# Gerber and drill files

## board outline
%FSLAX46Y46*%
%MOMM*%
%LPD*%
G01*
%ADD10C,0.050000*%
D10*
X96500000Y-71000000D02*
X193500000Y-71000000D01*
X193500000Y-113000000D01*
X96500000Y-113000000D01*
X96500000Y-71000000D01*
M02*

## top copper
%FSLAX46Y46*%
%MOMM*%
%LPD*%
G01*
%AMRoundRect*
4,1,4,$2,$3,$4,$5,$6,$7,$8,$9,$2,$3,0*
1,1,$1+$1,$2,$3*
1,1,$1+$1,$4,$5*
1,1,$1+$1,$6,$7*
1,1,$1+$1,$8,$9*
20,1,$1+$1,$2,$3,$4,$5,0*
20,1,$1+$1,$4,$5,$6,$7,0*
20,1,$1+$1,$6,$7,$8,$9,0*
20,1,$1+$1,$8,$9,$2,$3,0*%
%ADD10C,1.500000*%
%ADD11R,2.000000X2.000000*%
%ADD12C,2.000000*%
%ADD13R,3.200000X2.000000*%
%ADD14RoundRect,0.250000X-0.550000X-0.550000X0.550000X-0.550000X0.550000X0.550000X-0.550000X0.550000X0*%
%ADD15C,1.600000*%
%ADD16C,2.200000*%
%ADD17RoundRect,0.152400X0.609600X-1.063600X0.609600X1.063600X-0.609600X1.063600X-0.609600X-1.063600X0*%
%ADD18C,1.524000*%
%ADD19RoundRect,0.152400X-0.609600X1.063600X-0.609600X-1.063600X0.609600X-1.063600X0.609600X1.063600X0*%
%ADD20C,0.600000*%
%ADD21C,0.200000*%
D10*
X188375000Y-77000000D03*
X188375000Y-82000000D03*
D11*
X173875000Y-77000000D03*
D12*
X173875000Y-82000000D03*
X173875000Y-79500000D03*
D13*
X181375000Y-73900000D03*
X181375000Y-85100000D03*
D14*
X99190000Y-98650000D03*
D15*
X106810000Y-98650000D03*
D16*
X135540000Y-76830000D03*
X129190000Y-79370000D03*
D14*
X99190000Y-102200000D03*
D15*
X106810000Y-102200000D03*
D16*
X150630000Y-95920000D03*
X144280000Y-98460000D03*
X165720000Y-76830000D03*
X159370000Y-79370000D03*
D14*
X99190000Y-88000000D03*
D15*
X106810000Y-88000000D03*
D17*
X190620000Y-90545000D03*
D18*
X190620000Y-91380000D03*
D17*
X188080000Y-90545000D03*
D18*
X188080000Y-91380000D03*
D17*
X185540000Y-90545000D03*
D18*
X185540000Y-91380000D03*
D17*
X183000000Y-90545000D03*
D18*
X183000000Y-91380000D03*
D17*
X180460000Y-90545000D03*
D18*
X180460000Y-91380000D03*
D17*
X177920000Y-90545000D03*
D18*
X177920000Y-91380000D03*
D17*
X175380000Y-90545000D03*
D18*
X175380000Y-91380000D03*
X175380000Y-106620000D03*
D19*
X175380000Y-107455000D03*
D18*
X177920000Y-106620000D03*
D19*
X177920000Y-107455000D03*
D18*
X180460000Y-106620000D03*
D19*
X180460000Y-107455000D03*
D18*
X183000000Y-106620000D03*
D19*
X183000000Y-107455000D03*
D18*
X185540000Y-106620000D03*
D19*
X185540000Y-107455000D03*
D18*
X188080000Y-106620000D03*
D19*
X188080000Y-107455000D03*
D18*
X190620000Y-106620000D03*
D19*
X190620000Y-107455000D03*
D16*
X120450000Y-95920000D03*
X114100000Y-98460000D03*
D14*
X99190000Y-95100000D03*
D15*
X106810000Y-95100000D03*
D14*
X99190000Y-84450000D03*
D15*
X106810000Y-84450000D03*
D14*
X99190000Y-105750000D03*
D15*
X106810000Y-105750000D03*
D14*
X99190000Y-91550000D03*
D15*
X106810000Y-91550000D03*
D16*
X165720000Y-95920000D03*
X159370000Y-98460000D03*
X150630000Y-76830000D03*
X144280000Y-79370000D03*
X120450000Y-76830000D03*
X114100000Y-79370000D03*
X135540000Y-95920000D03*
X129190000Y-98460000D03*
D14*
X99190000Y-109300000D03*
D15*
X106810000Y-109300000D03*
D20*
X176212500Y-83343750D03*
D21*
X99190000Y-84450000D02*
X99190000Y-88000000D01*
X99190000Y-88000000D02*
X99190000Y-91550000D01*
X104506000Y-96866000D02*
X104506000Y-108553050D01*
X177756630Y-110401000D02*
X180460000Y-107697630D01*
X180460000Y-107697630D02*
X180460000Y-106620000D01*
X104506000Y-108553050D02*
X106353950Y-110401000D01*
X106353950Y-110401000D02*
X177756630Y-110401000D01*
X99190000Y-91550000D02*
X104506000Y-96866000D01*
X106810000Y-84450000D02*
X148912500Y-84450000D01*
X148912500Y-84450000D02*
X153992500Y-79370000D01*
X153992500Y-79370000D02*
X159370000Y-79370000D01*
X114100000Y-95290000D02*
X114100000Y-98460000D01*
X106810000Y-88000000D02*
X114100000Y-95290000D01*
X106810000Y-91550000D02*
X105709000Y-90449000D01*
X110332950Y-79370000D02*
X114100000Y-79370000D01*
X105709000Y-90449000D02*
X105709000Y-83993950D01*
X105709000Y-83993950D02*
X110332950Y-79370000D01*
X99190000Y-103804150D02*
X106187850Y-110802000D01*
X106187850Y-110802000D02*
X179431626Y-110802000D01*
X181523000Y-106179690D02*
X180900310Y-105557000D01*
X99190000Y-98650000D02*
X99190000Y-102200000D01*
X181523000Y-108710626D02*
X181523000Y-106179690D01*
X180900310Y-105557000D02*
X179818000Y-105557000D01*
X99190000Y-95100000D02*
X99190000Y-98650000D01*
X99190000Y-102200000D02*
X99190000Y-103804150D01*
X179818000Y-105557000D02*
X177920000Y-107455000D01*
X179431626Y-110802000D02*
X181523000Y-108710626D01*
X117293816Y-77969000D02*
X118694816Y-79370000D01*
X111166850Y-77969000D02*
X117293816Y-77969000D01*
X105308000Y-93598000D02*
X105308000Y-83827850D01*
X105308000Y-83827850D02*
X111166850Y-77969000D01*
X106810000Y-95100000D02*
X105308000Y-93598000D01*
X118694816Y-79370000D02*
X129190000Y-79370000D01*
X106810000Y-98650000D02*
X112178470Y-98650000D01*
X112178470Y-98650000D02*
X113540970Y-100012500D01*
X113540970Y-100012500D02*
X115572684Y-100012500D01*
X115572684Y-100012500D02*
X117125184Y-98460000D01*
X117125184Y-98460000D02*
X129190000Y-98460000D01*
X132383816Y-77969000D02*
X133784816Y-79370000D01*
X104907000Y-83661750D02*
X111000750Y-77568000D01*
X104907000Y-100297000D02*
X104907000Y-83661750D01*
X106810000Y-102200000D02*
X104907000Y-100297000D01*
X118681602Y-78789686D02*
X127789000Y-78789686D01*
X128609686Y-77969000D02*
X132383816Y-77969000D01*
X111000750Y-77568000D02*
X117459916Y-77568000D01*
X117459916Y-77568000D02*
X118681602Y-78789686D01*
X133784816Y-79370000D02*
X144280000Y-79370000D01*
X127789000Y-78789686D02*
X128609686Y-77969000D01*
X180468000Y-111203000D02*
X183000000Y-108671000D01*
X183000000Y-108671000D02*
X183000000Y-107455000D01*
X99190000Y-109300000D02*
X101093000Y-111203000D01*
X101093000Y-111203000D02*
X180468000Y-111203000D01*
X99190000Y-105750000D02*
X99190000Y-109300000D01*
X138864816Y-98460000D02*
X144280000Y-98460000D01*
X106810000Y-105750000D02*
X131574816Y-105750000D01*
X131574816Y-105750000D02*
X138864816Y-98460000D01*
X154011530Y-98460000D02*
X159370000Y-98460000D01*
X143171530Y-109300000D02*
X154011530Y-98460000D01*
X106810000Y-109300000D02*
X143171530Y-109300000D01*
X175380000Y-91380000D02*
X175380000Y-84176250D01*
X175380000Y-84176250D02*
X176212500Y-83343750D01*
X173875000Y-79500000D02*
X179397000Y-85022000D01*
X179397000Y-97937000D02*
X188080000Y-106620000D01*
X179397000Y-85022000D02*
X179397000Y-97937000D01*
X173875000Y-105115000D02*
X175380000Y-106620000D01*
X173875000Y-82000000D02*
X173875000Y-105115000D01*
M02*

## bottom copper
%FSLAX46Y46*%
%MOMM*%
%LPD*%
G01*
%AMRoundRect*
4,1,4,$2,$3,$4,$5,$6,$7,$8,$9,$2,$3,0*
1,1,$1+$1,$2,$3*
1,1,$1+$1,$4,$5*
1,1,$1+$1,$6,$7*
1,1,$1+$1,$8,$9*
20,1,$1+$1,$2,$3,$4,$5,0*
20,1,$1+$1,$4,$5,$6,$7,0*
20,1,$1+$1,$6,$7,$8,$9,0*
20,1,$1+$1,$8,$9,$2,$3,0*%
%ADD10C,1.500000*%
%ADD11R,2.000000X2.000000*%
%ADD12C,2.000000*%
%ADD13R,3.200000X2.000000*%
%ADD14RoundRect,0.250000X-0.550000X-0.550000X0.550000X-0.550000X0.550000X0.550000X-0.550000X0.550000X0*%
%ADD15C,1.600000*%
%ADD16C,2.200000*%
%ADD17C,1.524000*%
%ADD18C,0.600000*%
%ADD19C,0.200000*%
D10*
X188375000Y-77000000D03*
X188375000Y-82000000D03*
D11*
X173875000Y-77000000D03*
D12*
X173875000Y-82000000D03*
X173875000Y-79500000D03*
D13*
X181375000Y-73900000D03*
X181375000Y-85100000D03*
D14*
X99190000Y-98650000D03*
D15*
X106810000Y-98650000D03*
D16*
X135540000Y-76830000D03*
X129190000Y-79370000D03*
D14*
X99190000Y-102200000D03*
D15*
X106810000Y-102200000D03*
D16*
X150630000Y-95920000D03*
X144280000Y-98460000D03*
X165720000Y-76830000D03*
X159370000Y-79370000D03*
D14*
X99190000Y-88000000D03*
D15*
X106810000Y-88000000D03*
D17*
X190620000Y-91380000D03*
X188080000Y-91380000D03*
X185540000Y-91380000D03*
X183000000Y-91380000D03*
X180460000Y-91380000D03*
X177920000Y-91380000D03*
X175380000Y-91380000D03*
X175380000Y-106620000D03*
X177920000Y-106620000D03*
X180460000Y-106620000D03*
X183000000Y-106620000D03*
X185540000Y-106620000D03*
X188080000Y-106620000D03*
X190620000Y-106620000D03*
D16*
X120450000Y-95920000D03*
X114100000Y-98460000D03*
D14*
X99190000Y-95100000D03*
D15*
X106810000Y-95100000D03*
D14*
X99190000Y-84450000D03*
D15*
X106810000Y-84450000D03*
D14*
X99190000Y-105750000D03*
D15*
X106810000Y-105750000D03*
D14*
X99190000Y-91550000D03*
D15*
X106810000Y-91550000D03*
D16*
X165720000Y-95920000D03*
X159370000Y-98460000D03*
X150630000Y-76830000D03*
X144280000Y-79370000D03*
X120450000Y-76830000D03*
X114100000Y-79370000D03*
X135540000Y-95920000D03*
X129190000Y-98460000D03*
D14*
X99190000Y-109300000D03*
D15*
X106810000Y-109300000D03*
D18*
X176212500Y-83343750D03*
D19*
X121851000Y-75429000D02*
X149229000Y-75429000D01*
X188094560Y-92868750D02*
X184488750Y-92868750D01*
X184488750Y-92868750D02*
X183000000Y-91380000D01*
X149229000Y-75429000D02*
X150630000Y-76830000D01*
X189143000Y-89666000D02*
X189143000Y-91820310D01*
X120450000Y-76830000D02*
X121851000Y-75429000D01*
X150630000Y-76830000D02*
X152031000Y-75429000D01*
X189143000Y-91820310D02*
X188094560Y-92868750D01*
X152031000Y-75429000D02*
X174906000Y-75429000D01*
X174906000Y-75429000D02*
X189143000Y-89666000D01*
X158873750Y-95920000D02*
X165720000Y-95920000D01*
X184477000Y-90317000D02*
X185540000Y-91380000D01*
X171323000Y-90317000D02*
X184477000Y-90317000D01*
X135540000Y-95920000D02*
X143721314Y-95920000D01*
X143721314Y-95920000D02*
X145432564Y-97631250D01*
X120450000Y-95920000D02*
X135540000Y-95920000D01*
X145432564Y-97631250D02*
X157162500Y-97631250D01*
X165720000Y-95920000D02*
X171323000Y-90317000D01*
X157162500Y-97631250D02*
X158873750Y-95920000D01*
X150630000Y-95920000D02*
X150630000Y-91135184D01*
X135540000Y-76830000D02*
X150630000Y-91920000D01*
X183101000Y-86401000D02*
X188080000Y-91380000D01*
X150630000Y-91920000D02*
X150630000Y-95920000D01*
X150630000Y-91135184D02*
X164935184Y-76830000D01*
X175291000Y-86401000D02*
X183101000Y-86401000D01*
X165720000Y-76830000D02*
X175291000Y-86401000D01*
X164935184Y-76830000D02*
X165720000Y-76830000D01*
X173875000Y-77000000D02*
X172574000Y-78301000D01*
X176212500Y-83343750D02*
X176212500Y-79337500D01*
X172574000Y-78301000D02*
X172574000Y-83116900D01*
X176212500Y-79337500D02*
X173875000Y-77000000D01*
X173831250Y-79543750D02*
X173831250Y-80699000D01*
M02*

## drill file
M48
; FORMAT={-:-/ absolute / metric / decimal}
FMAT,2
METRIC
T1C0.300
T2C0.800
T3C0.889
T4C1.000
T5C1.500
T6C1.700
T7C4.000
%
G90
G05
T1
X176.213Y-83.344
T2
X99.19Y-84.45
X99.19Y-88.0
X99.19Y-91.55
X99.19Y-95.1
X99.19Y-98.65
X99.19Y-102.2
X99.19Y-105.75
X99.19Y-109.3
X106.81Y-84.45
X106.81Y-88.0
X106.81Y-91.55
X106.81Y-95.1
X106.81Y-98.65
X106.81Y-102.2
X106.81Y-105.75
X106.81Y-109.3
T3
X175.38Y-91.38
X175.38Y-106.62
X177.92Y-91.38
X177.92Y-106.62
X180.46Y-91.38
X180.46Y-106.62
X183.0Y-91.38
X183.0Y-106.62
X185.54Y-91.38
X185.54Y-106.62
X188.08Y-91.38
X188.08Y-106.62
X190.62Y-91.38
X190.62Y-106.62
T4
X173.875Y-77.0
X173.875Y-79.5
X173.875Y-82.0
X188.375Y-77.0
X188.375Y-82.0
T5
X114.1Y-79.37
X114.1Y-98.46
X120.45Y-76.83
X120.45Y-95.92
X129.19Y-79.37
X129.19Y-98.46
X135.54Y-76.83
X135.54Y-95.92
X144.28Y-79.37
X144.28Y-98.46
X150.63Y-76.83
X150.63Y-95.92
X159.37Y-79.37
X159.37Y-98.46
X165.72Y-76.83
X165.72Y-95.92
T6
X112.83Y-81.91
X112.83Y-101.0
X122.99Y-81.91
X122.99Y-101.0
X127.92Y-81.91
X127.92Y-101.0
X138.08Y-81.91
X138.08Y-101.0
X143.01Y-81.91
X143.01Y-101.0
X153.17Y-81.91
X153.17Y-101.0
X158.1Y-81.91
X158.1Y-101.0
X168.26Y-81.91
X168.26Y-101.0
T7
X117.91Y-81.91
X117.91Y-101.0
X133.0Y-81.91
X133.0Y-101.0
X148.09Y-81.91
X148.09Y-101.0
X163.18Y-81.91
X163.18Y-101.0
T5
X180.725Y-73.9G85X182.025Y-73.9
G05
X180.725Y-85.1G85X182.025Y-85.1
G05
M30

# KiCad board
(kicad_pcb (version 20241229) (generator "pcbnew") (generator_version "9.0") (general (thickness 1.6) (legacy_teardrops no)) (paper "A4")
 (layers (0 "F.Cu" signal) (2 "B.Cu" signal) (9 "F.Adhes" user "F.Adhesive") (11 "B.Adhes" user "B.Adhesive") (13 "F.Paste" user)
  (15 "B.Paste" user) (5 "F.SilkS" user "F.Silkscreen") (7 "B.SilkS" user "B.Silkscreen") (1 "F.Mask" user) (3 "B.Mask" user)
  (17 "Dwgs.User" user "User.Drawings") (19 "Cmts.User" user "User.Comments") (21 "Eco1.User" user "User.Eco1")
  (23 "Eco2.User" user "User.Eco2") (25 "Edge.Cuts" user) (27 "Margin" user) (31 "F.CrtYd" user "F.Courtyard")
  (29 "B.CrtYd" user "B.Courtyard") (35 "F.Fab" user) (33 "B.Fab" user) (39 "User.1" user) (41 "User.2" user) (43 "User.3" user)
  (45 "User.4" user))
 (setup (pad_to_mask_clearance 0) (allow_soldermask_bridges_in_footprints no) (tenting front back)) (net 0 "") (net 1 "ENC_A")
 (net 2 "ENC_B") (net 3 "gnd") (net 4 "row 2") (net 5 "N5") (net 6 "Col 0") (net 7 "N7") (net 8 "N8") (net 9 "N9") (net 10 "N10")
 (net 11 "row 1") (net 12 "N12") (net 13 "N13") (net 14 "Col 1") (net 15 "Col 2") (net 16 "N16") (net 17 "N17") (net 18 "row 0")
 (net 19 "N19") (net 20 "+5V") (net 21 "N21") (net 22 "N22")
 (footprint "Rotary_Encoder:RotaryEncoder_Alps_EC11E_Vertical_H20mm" (layer "F.Cu") (at 173.875 77)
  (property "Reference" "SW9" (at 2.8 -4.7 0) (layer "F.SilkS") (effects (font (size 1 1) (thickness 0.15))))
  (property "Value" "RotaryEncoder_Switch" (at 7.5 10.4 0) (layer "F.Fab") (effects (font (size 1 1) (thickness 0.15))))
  (pad "" thru_hole circle (at 14.5 0) (size 1.5 1.5) (drill 1) (layers "*.Cu" "*.Mask") (remove_unused_layers no))
  (pad "" thru_hole circle (at 14.5 5) (size 1.5 1.5) (drill 1) (layers "*.Cu" "*.Mask") (remove_unused_layers no))
  (pad "A" thru_hole rect (at 0 0) (size 2 2) (drill 1) (layers "*.Cu" "*.Mask") (remove_unused_layers no) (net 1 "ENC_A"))
  (pad "B" thru_hole circle (at 0 5) (size 2 2) (drill 1) (layers "*.Cu" "*.Mask") (remove_unused_layers no) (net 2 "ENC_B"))
  (pad "C" thru_hole circle (at 0 2.5) (size 2 2) (drill 1) (layers "*.Cu" "*.Mask") (remove_unused_layers no) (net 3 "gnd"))
  (pad "MP" thru_hole rect (at 7.5 -3.1) (size 3.2 2) (drill oval 2.8 1.5) (layers "*.Cu" "*.Mask") (remove_unused_layers no))
  (pad "MP" thru_hole rect (at 7.5 8.1) (size 3.2 2) (drill oval 2.8 1.5) (layers "*.Cu" "*.Mask") (remove_unused_layers no)))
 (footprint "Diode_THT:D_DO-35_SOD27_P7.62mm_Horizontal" (layer "F.Cu") (at 99.19 98.65)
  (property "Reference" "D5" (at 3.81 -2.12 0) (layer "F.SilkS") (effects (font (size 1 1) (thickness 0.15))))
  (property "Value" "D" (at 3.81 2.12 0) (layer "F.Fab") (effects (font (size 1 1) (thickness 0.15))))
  (pad "1" thru_hole roundrect (at 0 0) (size 1.6 1.6) (drill 0.8) (layers "*.Cu" "*.Mask") (remove_unused_layers no)
   (roundrect_rratio 0.15625) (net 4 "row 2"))
  (pad "2" thru_hole circle (at 7.62 0) (size 1.6 1.6) (drill 0.8) (layers "*.Cu" "*.Mask") (remove_unused_layers no) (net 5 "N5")))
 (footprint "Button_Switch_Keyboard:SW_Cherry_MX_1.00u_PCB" (layer "F.Cu") (at 135.54 76.83)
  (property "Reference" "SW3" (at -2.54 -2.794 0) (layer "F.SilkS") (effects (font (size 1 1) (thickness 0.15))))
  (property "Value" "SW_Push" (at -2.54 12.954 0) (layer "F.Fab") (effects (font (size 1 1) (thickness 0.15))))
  (pad "" np_thru_hole circle (at -7.62 5.08) (size 1.7 1.7) (drill 1.7) (layers "*.Cu" "*.Mask"))
  (pad "" np_thru_hole circle (at -2.54 5.08) (size 4 4) (drill 4) (layers "*.Cu" "*.Mask"))
  (pad "" np_thru_hole circle (at 2.54 5.08) (size 1.7 1.7) (drill 1.7) (layers "*.Cu" "*.Mask"))
  (pad "1" thru_hole circle (at 0 0) (size 2.2 2.2) (drill 1.5) (layers "*.Cu" "*.Mask") (remove_unused_layers no) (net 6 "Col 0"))
  (pad "2" thru_hole circle (at -6.35 2.54) (size 2.2 2.2) (drill 1.5) (layers "*.Cu" "*.Mask") (remove_unused_layers no) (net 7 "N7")))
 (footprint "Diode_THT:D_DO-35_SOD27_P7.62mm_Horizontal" (layer "F.Cu") (at 99.19 102.2)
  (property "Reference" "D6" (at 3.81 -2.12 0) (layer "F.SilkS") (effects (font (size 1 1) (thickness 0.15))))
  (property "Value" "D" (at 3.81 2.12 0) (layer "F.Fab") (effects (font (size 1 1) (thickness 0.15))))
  (pad "1" thru_hole roundrect (at 0 0) (size 1.6 1.6) (drill 0.8) (layers "*.Cu" "*.Mask") (remove_unused_layers no)
   (roundrect_rratio 0.15625) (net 4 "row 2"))
  (pad "2" thru_hole circle (at 7.62 0) (size 1.6 1.6) (drill 0.8) (layers "*.Cu" "*.Mask") (remove_unused_layers no) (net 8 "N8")))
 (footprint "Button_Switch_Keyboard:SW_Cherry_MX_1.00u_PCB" (layer "F.Cu") (at 150.63 95.92)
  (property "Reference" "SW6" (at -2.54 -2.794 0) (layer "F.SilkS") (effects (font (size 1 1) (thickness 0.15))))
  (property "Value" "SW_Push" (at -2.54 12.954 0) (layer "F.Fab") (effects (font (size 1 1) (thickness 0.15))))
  (pad "" np_thru_hole circle (at -7.62 5.08) (size 1.7 1.7) (drill 1.7) (layers "*.Cu" "*.Mask"))
  (pad "" np_thru_hole circle (at -2.54 5.08) (size 4 4) (drill 4) (layers "*.Cu" "*.Mask"))
  (pad "" np_thru_hole circle (at 2.54 5.08) (size 1.7 1.7) (drill 1.7) (layers "*.Cu" "*.Mask"))
  (pad "1" thru_hole circle (at 0 0) (size 2.2 2.2) (drill 1.5) (layers "*.Cu" "*.Mask") (remove_unused_layers no) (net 6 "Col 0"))
  (pad "2" thru_hole circle (at -6.35 2.54) (size 2.2 2.2) (drill 1.5) (layers "*.Cu" "*.Mask") (remove_unused_layers no) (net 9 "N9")))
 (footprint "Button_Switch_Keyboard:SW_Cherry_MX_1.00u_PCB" (layer "F.Cu") (at 165.72 76.83)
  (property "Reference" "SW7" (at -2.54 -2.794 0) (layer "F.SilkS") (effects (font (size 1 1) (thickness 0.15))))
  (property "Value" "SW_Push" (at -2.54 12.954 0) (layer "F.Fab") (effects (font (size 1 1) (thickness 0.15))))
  (pad "" np_thru_hole circle (at -7.62 5.08) (size 1.7 1.7) (drill 1.7) (layers "*.Cu" "*.Mask"))
  (pad "" np_thru_hole circle (at -2.54 5.08) (size 4 4) (drill 4) (layers "*.Cu" "*.Mask"))
  (pad "" np_thru_hole circle (at 2.54 5.08) (size 1.7 1.7) (drill 1.7) (layers "*.Cu" "*.Mask"))
  (pad "1" thru_hole circle (at 0 0) (size 2.2 2.2) (drill 1.5) (layers "*.Cu" "*.Mask") (remove_unused_layers no) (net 6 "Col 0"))
  (pad "2" thru_hole circle (at -6.35 2.54) (size 2.2 2.2) (drill 1.5) (layers "*.Cu" "*.Mask") (remove_unused_layers no) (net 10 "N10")))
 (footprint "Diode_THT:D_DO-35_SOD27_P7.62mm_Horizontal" (layer "F.Cu") (at 99.19 88)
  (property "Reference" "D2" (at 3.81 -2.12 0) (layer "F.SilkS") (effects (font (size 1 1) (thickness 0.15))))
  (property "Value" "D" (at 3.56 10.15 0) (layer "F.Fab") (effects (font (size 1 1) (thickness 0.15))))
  (pad "1" thru_hole roundrect (at 0 0) (size 1.6 1.6) (drill 0.8) (layers "*.Cu" "*.Mask") (remove_unused_layers no)
   (roundrect_rratio 0.15625) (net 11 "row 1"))
  (pad "2" thru_hole circle (at 7.62 0) (size 1.6 1.6) (drill 0.8) (layers "*.Cu" "*.Mask") (remove_unused_layers no) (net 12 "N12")))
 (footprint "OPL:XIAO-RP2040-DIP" (layer "F.Cu") (at 183 99 -90)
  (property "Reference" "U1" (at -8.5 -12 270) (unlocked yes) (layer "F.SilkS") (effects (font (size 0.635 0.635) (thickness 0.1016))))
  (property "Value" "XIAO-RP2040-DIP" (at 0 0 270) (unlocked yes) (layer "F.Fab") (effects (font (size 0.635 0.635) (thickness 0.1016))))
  (pad "1" smd roundrect (at -8.455 -7.62 90) (size 2.432 1.524) (layers "F.Cu" "F.Mask") (roundrect_rratio 0.1) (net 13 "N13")
   (thermal_bridge_angle 45))
  (pad "1" thru_hole circle (at -7.62 -7.62 90) (size 1.524 1.524) (drill 0.889) (layers "*.Cu" "*.Mask") (remove_unused_layers no)
   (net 13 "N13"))
  (pad "2" smd roundrect (at -8.455 -5.08 90) (size 2.432 1.524) (layers "F.Cu" "F.Mask") (roundrect_rratio 0.1) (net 6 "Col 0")
   (thermal_bridge_angle 45))
  (pad "2" thru_hole circle (at -7.62 -5.08 90) (size 1.524 1.524) (drill 0.889) (layers "*.Cu" "*.Mask") (remove_unused_layers no)
   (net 6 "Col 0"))
  (pad "3" smd roundrect (at -8.455 -2.54 90) (size 2.432 1.524) (layers "F.Cu" "F.Mask") (roundrect_rratio 0.1) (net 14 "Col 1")
   (thermal_bridge_angle 45))
  (pad "3" thru_hole circle (at -7.62 -2.54 90) (size 1.524 1.524) (drill 0.889) (layers "*.Cu" "*.Mask") (remove_unused_layers no)
   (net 14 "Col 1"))
  (pad "4" smd roundrect (at -8.455 0 90) (size 2.432 1.524) (layers "F.Cu" "F.Mask") (roundrect_rratio 0.1) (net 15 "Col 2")
   (thermal_bridge_angle 45))
  (pad "4" thru_hole circle (at -7.62 0 90) (size 1.524 1.524) (drill 0.889) (layers "*.Cu" "*.Mask") (remove_unused_layers no)
   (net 15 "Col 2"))
  (pad "5" smd roundrect (at -8.455 2.54 90) (size 2.432 1.524) (layers "F.Cu" "F.Mask") (roundrect_rratio 0.1) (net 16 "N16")
   (thermal_bridge_angle 45))
  (pad "5" thru_hole circle (at -7.62 2.54 90) (size 1.524 1.524) (drill 0.889) (layers "*.Cu" "*.Mask") (remove_unused_layers no)
   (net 16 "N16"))
  (pad "6" smd roundrect (at -8.455 5.08 90) (size 2.432 1.524) (layers "F.Cu" "F.Mask") (roundrect_rratio 0.1) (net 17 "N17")
   (thermal_bridge_angle 45))
  (pad "6" thru_hole circle (at -7.62 5.08 90) (size 1.524 1.524) (drill 0.889) (layers "*.Cu" "*.Mask") (remove_unused_layers no)
   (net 17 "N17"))
  (pad "7" smd roundrect (at -8.455 7.62 90) (size 2.432 1.524) (layers "F.Cu" "F.Mask") (roundrect_rratio 0.1) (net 1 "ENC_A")
   (thermal_bridge_angle 45))
  (pad "7" thru_hole circle (at -7.62 7.62 90) (size 1.524 1.524) (drill 0.889) (layers "*.Cu" "*.Mask") (remove_unused_layers no)
   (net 1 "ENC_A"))
  (pad "8" thru_hole circle (at 7.62 7.62 270) (size 1.524 1.524) (drill 0.889) (layers "*.Cu" "*.Mask") (remove_unused_layers no)
   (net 2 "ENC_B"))
  (pad "8" smd roundrect (at 8.455 7.62 270) (size 2.432 1.524) (layers "F.Cu" "F.Mask") (roundrect_rratio 0.1) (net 2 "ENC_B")
   (thermal_bridge_angle 45))
  (pad "9" thru_hole circle (at 7.62 5.08 270) (size 1.524 1.524) (drill 0.889) (layers "*.Cu" "*.Mask") (remove_unused_layers no)
   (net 4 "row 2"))
  (pad "9" smd roundrect (at 8.455 5.08 270) (size 2.432 1.524) (layers "F.Cu" "F.Mask") (roundrect_rratio 0.1) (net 4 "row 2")
   (thermal_bridge_angle 45))
  (pad "10" thru_hole circle (at 7.62 2.54 270) (size 1.524 1.524) (drill 0.889) (layers "*.Cu" "*.Mask") (remove_unused_layers no)
   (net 11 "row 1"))
  (pad "10" smd roundrect (at 8.455 2.54 270) (size 2.432 1.524) (layers "F.Cu" "F.Mask") (roundrect_rratio 0.1) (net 11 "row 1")
   (thermal_bridge_angle 45))
  (pad "11" thru_hole circle (at 7.62 0 270) (size 1.524 1.524) (drill 0.889) (layers "*.Cu" "*.Mask") (remove_unused_layers no)
   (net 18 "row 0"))
  (pad "11" smd roundrect (at 8.455 0 270) (size 2.432 1.524) (layers "F.Cu" "F.Mask") (roundrect_rratio 0.1) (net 18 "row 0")
   (thermal_bridge_angle 45))
  (pad "12" thru_hole circle (at 7.62 -2.54 270) (size 1.524 1.524) (drill 0.889) (layers "*.Cu" "*.Mask") (remove_unused_layers no)
   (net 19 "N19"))
  (pad "12" smd roundrect (at 8.455 -2.54 270) (size 2.432 1.524) (layers "F.Cu" "F.Mask") (roundrect_rratio 0.1) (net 19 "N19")
   (thermal_bridge_angle 45))
  (pad "13" thru_hole circle (at 7.62 -5.08 270) (size 1.524 1.524) (drill 0.889) (layers "*.Cu" "*.Mask") (remove_unused_layers no)
   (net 3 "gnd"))
  (pad "13" smd roundrect (at 8.455 -5.08 270) (size 2.432 1.524) (layers "F.Cu" "F.Mask") (roundrect_rratio 0.1) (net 3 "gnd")
   (thermal_bridge_angle 45))
  (pad "14" thru_hole circle (at 7.62 -7.62 270) (size 1.524 1.524) (drill 0.889) (layers "*.Cu" "*.Mask") (remove_unused_layers no)
   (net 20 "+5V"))
  (pad "14" smd roundrect (at 8.455 -7.62 270) (size 2.432 1.524) (layers "F.Cu" "F.Mask") (roundrect_rratio 0.1) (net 20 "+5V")
   (thermal_bridge_angle 45)))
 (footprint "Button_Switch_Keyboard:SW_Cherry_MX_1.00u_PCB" (layer "F.Cu") (at 120.45 95.92)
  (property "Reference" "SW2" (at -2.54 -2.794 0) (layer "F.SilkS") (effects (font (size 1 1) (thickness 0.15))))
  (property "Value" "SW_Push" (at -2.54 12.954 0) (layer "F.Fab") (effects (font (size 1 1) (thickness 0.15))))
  (pad "" np_thru_hole circle (at -7.62 5.08) (size 1.7 1.7) (drill 1.7) (layers "*.Cu" "*.Mask"))
  (pad "" np_thru_hole circle (at -2.54 5.08) (size 4 4) (drill 4) (layers "*.Cu" "*.Mask"))
  (pad "" np_thru_hole circle (at 2.54 5.08) (size 1.7 1.7) (drill 1.7) (layers "*.Cu" "*.Mask"))
  (pad "1" thru_hole circle (at 0 0) (size 2.2 2.2) (drill 1.5) (layers "*.Cu" "*.Mask") (remove_unused_layers no) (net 14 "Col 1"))
  (pad "2" thru_hole circle (at -6.35 2.54) (size 2.2 2.2) (drill 1.5) (layers "*.Cu" "*.Mask") (remove_unused_layers no) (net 12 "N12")))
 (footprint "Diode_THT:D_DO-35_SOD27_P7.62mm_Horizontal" (layer "F.Cu") (at 99.19 95.1)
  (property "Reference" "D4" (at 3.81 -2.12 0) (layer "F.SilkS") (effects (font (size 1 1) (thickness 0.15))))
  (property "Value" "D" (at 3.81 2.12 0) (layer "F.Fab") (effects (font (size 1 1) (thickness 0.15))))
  (pad "1" thru_hole roundrect (at 0 0) (size 1.6 1.6) (drill 0.8) (layers "*.Cu" "*.Mask") (remove_unused_layers no)
   (roundrect_rratio 0.15625) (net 4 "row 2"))
  (pad "2" thru_hole circle (at 7.62 0) (size 1.6 1.6) (drill 0.8) (layers "*.Cu" "*.Mask") (remove_unused_layers no) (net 7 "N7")))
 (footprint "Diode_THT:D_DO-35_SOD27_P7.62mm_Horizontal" (layer "F.Cu") (at 99.19 84.45)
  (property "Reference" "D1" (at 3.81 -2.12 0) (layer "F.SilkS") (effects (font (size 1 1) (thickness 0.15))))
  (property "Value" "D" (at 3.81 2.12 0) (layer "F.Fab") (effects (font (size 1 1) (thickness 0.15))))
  (pad "1" thru_hole roundrect (at 0 0) (size 1.6 1.6) (drill 0.8) (layers "*.Cu" "*.Mask") (remove_unused_layers no)
   (roundrect_rratio 0.15625) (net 11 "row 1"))
  (pad "2" thru_hole circle (at 7.62 0) (size 1.6 1.6) (drill 0.8) (layers "*.Cu" "*.Mask") (remove_unused_layers no) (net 10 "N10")))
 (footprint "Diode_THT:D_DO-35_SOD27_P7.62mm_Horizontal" (layer "F.Cu") (at 99.19 105.75)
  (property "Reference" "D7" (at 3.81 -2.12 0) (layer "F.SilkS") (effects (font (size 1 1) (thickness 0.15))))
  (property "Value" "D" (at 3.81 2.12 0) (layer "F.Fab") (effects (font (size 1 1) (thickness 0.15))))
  (pad "1" thru_hole roundrect (at 0 0) (size 1.6 1.6) (drill 0.8) (layers "*.Cu" "*.Mask") (remove_unused_layers no)
   (roundrect_rratio 0.15625) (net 18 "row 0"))
  (pad "2" thru_hole circle (at 7.62 0) (size 1.6 1.6) (drill 0.8) (layers "*.Cu" "*.Mask") (remove_unused_layers no) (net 9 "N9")))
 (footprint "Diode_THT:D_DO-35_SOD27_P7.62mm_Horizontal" (layer "F.Cu") (at 99.19 91.55)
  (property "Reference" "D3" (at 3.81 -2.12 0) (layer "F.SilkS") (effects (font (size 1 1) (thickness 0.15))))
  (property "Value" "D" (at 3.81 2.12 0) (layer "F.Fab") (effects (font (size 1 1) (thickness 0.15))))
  (pad "1" thru_hole roundrect (at 0 0) (size 1.6 1.6) (drill 0.8) (layers "*.Cu" "*.Mask") (remove_unused_layers no)
   (roundrect_rratio 0.15625) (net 11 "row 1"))
  (pad "2" thru_hole circle (at 7.62 0) (size 1.6 1.6) (drill 0.8) (layers "*.Cu" "*.Mask") (remove_unused_layers no) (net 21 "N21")))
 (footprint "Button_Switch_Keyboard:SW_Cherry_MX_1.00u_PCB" (layer "F.Cu") (at 165.72 95.92)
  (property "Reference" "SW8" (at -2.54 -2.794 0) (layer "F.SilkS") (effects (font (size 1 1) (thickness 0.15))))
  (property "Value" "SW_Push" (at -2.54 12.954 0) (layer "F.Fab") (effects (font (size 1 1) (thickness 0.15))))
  (pad "" np_thru_hole circle (at -7.62 5.08) (size 1.7 1.7) (drill 1.7) (layers "*.Cu" "*.Mask"))
  (pad "" np_thru_hole circle (at -2.54 5.08) (size 4 4) (drill 4) (layers "*.Cu" "*.Mask"))
  (pad "" np_thru_hole circle (at 2.54 5.08) (size 1.7 1.7) (drill 1.7) (layers "*.Cu" "*.Mask"))
  (pad "1" thru_hole circle (at 0 0) (size 2.2 2.2) (drill 1.5) (layers "*.Cu" "*.Mask") (remove_unused_layers no) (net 14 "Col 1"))
  (pad "2" thru_hole circle (at -6.35 2.54) (size 2.2 2.2) (drill 1.5) (layers "*.Cu" "*.Mask") (remove_unused_layers no) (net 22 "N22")))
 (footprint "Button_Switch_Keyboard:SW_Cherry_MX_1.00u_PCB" (layer "F.Cu") (at 150.63 76.83)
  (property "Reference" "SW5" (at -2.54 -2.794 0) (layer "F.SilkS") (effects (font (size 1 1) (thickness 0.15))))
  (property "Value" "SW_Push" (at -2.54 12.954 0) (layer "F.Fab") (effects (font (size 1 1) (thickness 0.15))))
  (pad "" np_thru_hole circle (at -7.62 5.08) (size 1.7 1.7) (drill 1.7) (layers "*.Cu" "*.Mask"))
  (pad "" np_thru_hole circle (at -2.54 5.08) (size 4 4) (drill 4) (layers "*.Cu" "*.Mask"))
  (pad "" np_thru_hole circle (at 2.54 5.08) (size 1.7 1.7) (drill 1.7) (layers "*.Cu" "*.Mask"))
  (pad "1" thru_hole circle (at 0 0) (size 2.2 2.2) (drill 1.5) (layers "*.Cu" "*.Mask") (remove_unused_layers no) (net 15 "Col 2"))
  (pad "2" thru_hole circle (at -6.35 2.54) (size 2.2 2.2) (drill 1.5) (layers "*.Cu" "*.Mask") (remove_unused_layers no) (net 8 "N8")))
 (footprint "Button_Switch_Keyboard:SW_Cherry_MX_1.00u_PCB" (layer "F.Cu") (at 120.45 76.83)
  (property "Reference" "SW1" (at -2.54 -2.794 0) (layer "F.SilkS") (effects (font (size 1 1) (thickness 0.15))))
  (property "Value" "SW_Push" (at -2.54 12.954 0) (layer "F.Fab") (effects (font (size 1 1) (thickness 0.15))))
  (pad "" np_thru_hole circle (at -7.62 5.08) (size 1.7 1.7) (drill 1.7) (layers "*.Cu" "*.Mask"))
  (pad "" np_thru_hole circle (at -2.54 5.08) (size 4 4) (drill 4) (layers "*.Cu" "*.Mask"))
  (pad "" np_thru_hole circle (at 2.54 5.08) (size 1.7 1.7) (drill 1.7) (layers "*.Cu" "*.Mask"))
  (pad "1" thru_hole circle (at 0 0) (size 2.2 2.2) (drill 1.5) (layers "*.Cu" "*.Mask") (remove_unused_layers no) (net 15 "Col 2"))
  (pad "2" thru_hole circle (at -6.35 2.54) (size 2.2 2.2) (drill 1.5) (layers "*.Cu" "*.Mask") (remove_unused_layers no) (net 21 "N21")))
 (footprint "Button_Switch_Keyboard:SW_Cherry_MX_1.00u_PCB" (layer "F.Cu") (at 135.54 95.92)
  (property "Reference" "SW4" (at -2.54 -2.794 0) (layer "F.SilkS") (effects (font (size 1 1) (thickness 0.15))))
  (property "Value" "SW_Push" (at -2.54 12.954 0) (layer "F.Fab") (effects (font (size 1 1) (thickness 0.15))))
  (pad "" np_thru_hole circle (at -7.62 5.08) (size 1.7 1.7) (drill 1.7) (layers "*.Cu" "*.Mask"))
  (pad "" np_thru_hole circle (at -2.54 5.08) (size 4 4) (drill 4) (layers "*.Cu" "*.Mask"))
  (pad "" np_thru_hole circle (at 2.54 5.08) (size 1.7 1.7) (drill 1.7) (layers "*.Cu" "*.Mask"))
  (pad "1" thru_hole circle (at 0 0) (size 2.2 2.2) (drill 1.5) (layers "*.Cu" "*.Mask") (remove_unused_layers no) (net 14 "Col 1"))
  (pad "2" thru_hole circle (at -6.35 2.54) (size 2.2 2.2) (drill 1.5) (layers "*.Cu" "*.Mask") (remove_unused_layers no) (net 5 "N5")))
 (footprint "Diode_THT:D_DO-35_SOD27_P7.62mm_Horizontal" (layer "F.Cu") (at 99.19 109.3)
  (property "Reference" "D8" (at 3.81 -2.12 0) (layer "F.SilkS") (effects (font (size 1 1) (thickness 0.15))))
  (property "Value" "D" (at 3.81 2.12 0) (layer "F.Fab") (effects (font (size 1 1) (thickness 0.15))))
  (pad "1" thru_hole roundrect (at 0 0) (size 1.6 1.6) (drill 0.8) (layers "*.Cu" "*.Mask") (remove_unused_layers no)
   (roundrect_rratio 0.15625) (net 18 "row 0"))
  (pad "2" thru_hole circle (at 7.62 0) (size 1.6 1.6) (drill 0.8) (layers "*.Cu" "*.Mask") (remove_unused_layers no) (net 22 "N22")))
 (gr_rect (start 96.5 71) (end 193.5 113) (stroke (width 0.05) (type default)) (fill no) (layer "Edge.Cuts"))
 (segment (start 99.19 84.45) (end 99.19 88) (width 0.2) (layer "F.Cu") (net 11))
 (segment (start 99.19 88) (end 99.19 91.55) (width 0.2) (layer "F.Cu") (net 11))
 (segment (start 104.506 96.866) (end 104.506 108.55305) (width 0.2) (layer "F.Cu") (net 11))
 (segment (start 177.75663 110.401) (end 180.46 107.69763) (width 0.2) (layer "F.Cu") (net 11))
 (segment (start 180.46 107.69763) (end 180.46 106.62) (width 0.2) (layer "F.Cu") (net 11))
 (segment (start 104.506 108.55305) (end 106.35395 110.401) (width 0.2) (layer "F.Cu") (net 11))
 (segment (start 106.35395 110.401) (end 177.75663 110.401) (width 0.2) (layer "F.Cu") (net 11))
 (segment (start 99.19 91.55) (end 104.506 96.866) (width 0.2) (layer "F.Cu") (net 11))
 (segment (start 106.81 84.45) (end 148.9125 84.45) (width 0.2) (layer "F.Cu") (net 10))
 (segment (start 148.9125 84.45) (end 153.9925 79.37) (width 0.2) (layer "F.Cu") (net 10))
 (segment (start 153.9925 79.37) (end 159.37 79.37) (width 0.2) (layer "F.Cu") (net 10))
 (segment (start 114.1 95.29) (end 114.1 98.46) (width 0.2) (layer "F.Cu") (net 12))
 (segment (start 106.81 88) (end 114.1 95.29) (width 0.2) (layer "F.Cu") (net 12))
 (segment (start 106.81 91.55) (end 105.709 90.449) (width 0.2) (layer "F.Cu") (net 21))
 (segment (start 110.33295 79.37) (end 114.1 79.37) (width 0.2) (layer "F.Cu") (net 21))
 (segment (start 105.709 90.449) (end 105.709 83.99395) (width 0.2) (layer "F.Cu") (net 21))
 (segment (start 105.709 83.99395) (end 110.33295 79.37) (width 0.2) (layer "F.Cu") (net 21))
 (segment (start 99.19 103.80415) (end 106.18785 110.802) (width 0.2) (layer "F.Cu") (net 4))
 (segment (start 106.18785 110.802) (end 179.431626 110.802) (width 0.2) (layer "F.Cu") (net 4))
 (segment (start 181.523 106.17969) (end 180.90031 105.557) (width 0.2) (layer "F.Cu") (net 4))
 (segment (start 99.19 98.65) (end 99.19 102.2) (width 0.2) (layer "F.Cu") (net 4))
 (segment (start 181.523 108.710626) (end 181.523 106.17969) (width 0.2) (layer "F.Cu") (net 4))
 (segment (start 180.90031 105.557) (end 179.818 105.557) (width 0.2) (layer "F.Cu") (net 4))
 (segment (start 99.19 95.1) (end 99.19 98.65) (width 0.2) (layer "F.Cu") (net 4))
 (segment (start 99.19 102.2) (end 99.19 103.80415) (width 0.2) (layer "F.Cu") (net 4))
 (segment (start 179.818 105.557) (end 177.92 107.455) (width 0.2) (layer "F.Cu") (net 4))
 (segment (start 179.431626 110.802) (end 181.523 108.710626) (width 0.2) (layer "F.Cu") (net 4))
 (segment (start 117.293816 77.969) (end 118.694816 79.37) (width 0.2) (layer "F.Cu") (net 7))
 (segment (start 111.16685 77.969) (end 117.293816 77.969) (width 0.2) (layer "F.Cu") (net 7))
 (segment (start 105.308 93.598) (end 105.308 83.82785) (width 0.2) (layer "F.Cu") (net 7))
 (segment (start 105.308 83.82785) (end 111.16685 77.969) (width 0.2) (layer "F.Cu") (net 7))
 (segment (start 106.81 95.1) (end 105.308 93.598) (width 0.2) (layer "F.Cu") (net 7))
 (segment (start 118.694816 79.37) (end 129.19 79.37) (width 0.2) (layer "F.Cu") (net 7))
 (segment (start 106.81 98.65) (end 112.17847 98.65) (width 0.2) (layer "F.Cu") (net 5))
 (segment (start 112.17847 98.65) (end 113.54097 100.0125) (width 0.2) (layer "F.Cu") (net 5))
 (segment (start 113.54097 100.0125) (end 115.572684 100.0125) (width 0.2) (layer "F.Cu") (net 5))
 (segment (start 115.572684 100.0125) (end 117.125184 98.46) (width 0.2) (layer "F.Cu") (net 5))
 (segment (start 117.125184 98.46) (end 129.19 98.46) (width 0.2) (layer "F.Cu") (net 5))
 (segment (start 132.383816 77.969) (end 133.784816 79.37) (width 0.2) (layer "F.Cu") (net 8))
 (segment (start 104.907 83.66175) (end 111.00075 77.568) (width 0.2) (layer "F.Cu") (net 8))
 (segment (start 104.907 100.297) (end 104.907 83.66175) (width 0.2) (layer "F.Cu") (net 8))
 (segment (start 106.81 102.2) (end 104.907 100.297) (width 0.2) (layer "F.Cu") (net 8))
 (segment (start 118.681602 78.789686) (end 127.789 78.789686) (width 0.2) (layer "F.Cu") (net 8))
 (segment (start 128.609686 77.969) (end 132.383816 77.969) (width 0.2) (layer "F.Cu") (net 8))
 (segment (start 111.00075 77.568) (end 117.459916 77.568) (width 0.2) (layer "F.Cu") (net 8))
 (segment (start 117.459916 77.568) (end 118.681602 78.789686) (width 0.2) (layer "F.Cu") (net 8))
 (segment (start 133.784816 79.37) (end 144.28 79.37) (width 0.2) (layer "F.Cu") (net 8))
 (segment (start 127.789 78.789686) (end 128.609686 77.969) (width 0.2) (layer "F.Cu") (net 8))
 (segment (start 180.468 111.203) (end 183 108.671) (width 0.2) (layer "F.Cu") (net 18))
 (segment (start 183 108.671) (end 183 107.455) (width 0.2) (layer "F.Cu") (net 18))
 (segment (start 99.19 109.3) (end 101.093 111.203) (width 0.2) (layer "F.Cu") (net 18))
 (segment (start 101.093 111.203) (end 180.468 111.203) (width 0.2) (layer "F.Cu") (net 18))
 (segment (start 99.19 105.75) (end 99.19 109.3) (width 0.2) (layer "F.Cu") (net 18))
 (segment (start 138.864816 98.46) (end 144.28 98.46) (width 0.2) (layer "F.Cu") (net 9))
 (segment (start 106.81 105.75) (end 131.574816 105.75) (width 0.2) (layer "F.Cu") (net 9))
 (segment (start 131.574816 105.75) (end 138.864816 98.46) (width 0.2) (layer "F.Cu") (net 9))
 (segment (start 154.01153 98.46) (end 159.37 98.46) (width 0.2) (layer "F.Cu") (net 22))
 (segment (start 143.17153 109.3) (end 154.01153 98.46) (width 0.2) (layer "F.Cu") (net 22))
 (segment (start 106.81 109.3) (end 143.17153 109.3) (width 0.2) (layer "F.Cu") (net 22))
 (segment (start 121.851 75.429) (end 149.229 75.429) (width 0.2) (layer "B.Cu") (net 15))
 (segment (start 188.09456 92.86875) (end 184.48875 92.86875) (width 0.2) (layer "B.Cu") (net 15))
 (segment (start 184.48875 92.86875) (end 183 91.38) (width 0.2) (layer "B.Cu") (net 15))
 (segment (start 149.229 75.429) (end 150.63 76.83) (width 0.2) (layer "B.Cu") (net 15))
 (segment (start 189.143 89.666) (end 189.143 91.82031) (width 0.2) (layer "B.Cu") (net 15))
 (segment (start 120.45 76.83) (end 121.851 75.429) (width 0.2) (layer "B.Cu") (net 15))
 (segment (start 150.63 76.83) (end 152.031 75.429) (width 0.2) (layer "B.Cu") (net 15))
 (segment (start 189.143 91.82031) (end 188.09456 92.86875) (width 0.2) (layer "B.Cu") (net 15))
 (segment (start 152.031 75.429) (end 174.906 75.429) (width 0.2) (layer "B.Cu") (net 15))
 (segment (start 174.906 75.429) (end 189.143 89.666) (width 0.2) (layer "B.Cu") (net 15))
 (segment (start 158.87375 95.92) (end 165.72 95.92) (width 0.2) (layer "B.Cu") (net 14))
 (segment (start 184.477 90.317) (end 185.54 91.38) (width 0.2) (layer "B.Cu") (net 14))
 (segment (start 171.323 90.317) (end 184.477 90.317) (width 0.2) (layer "B.Cu") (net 14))
 (segment (start 135.54 95.92) (end 143.721314 95.92) (width 0.2) (layer "B.Cu") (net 14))
 (segment (start 143.721314 95.92) (end 145.432564 97.63125) (width 0.2) (layer "B.Cu") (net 14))
 (segment (start 120.45 95.92) (end 135.54 95.92) (width 0.2) (layer "B.Cu") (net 14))
 (segment (start 145.432564 97.63125) (end 157.1625 97.63125) (width 0.2) (layer "B.Cu") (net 14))
 (segment (start 165.72 95.92) (end 171.323 90.317) (width 0.2) (layer "B.Cu") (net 14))
 (segment (start 157.1625 97.63125) (end 158.87375 95.92) (width 0.2) (layer "B.Cu") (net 14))
 (segment (start 150.63 95.92) (end 150.63 91.135184) (width 0.2) (layer "B.Cu") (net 6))
 (segment (start 135.54 76.83) (end 150.63 91.92) (width 0.2) (layer "B.Cu") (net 6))
 (segment (start 183.101 86.401) (end 188.08 91.38) (width 0.2) (layer "B.Cu") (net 6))
 (segment (start 150.63 91.92) (end 150.63 95.92) (width 0.2) (layer "B.Cu") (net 6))
 (segment (start 150.63 91.135184) (end 164.935184 76.83) (width 0.2) (layer "B.Cu") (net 6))
 (segment (start 175.291 86.401) (end 183.101 86.401) (width 0.2) (layer "B.Cu") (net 6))
 (segment (start 165.72 76.83) (end 175.291 86.401) (width 0.2) (layer "B.Cu") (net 6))
 (segment (start 164.935184 76.83) (end 165.72 76.83) (width 0.2) (layer "B.Cu") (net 6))
 (segment (start 175.38 91.38) (end 175.38 84.17625) (width 0.2) (layer "F.Cu") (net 1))
 (segment (start 175.38 84.17625) (end 176.2125 83.34375) (width 0.2) (layer "F.Cu") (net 1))
 (via (at 176.2125 83.34375) (size 0.6) (drill 0.3) (layers "F.Cu" "B.Cu") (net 1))
 (segment (start 173.875 77) (end 172.574 78.301) (width 0.2) (layer "B.Cu") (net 1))
 (segment (start 176.2125 83.34375) (end 176.2125 79.3375) (width 0.2) (layer "B.Cu") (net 1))
 (segment (start 172.574 78.301) (end 172.574 83.1169) (width 0.2) (layer "B.Cu") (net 1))
 (segment (start 176.2125 79.3375) (end 173.875 77) (width 0.2) (layer "B.Cu") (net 1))
 (segment (start 173.875 79.5) (end 179.397 85.022) (width 0.2) (layer "F.Cu") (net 3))
 (segment (start 179.397 97.937) (end 188.08 106.62) (width 0.2) (layer "F.Cu") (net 3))
 (segment (start 179.397 85.022) (end 179.397 97.937) (width 0.2) (layer "F.Cu") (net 3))
 (segment (start 173.83125 79.54375) (end 173.83125 80.699) (width 0.2) (layer "B.Cu") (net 3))
 (segment (start 173.875 105.115) (end 175.38 106.62) (width 0.2) (layer "F.Cu") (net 2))
 (segment (start 173.875 82) (end 173.875 105.115) (width 0.2) (layer "F.Cu") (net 2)))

